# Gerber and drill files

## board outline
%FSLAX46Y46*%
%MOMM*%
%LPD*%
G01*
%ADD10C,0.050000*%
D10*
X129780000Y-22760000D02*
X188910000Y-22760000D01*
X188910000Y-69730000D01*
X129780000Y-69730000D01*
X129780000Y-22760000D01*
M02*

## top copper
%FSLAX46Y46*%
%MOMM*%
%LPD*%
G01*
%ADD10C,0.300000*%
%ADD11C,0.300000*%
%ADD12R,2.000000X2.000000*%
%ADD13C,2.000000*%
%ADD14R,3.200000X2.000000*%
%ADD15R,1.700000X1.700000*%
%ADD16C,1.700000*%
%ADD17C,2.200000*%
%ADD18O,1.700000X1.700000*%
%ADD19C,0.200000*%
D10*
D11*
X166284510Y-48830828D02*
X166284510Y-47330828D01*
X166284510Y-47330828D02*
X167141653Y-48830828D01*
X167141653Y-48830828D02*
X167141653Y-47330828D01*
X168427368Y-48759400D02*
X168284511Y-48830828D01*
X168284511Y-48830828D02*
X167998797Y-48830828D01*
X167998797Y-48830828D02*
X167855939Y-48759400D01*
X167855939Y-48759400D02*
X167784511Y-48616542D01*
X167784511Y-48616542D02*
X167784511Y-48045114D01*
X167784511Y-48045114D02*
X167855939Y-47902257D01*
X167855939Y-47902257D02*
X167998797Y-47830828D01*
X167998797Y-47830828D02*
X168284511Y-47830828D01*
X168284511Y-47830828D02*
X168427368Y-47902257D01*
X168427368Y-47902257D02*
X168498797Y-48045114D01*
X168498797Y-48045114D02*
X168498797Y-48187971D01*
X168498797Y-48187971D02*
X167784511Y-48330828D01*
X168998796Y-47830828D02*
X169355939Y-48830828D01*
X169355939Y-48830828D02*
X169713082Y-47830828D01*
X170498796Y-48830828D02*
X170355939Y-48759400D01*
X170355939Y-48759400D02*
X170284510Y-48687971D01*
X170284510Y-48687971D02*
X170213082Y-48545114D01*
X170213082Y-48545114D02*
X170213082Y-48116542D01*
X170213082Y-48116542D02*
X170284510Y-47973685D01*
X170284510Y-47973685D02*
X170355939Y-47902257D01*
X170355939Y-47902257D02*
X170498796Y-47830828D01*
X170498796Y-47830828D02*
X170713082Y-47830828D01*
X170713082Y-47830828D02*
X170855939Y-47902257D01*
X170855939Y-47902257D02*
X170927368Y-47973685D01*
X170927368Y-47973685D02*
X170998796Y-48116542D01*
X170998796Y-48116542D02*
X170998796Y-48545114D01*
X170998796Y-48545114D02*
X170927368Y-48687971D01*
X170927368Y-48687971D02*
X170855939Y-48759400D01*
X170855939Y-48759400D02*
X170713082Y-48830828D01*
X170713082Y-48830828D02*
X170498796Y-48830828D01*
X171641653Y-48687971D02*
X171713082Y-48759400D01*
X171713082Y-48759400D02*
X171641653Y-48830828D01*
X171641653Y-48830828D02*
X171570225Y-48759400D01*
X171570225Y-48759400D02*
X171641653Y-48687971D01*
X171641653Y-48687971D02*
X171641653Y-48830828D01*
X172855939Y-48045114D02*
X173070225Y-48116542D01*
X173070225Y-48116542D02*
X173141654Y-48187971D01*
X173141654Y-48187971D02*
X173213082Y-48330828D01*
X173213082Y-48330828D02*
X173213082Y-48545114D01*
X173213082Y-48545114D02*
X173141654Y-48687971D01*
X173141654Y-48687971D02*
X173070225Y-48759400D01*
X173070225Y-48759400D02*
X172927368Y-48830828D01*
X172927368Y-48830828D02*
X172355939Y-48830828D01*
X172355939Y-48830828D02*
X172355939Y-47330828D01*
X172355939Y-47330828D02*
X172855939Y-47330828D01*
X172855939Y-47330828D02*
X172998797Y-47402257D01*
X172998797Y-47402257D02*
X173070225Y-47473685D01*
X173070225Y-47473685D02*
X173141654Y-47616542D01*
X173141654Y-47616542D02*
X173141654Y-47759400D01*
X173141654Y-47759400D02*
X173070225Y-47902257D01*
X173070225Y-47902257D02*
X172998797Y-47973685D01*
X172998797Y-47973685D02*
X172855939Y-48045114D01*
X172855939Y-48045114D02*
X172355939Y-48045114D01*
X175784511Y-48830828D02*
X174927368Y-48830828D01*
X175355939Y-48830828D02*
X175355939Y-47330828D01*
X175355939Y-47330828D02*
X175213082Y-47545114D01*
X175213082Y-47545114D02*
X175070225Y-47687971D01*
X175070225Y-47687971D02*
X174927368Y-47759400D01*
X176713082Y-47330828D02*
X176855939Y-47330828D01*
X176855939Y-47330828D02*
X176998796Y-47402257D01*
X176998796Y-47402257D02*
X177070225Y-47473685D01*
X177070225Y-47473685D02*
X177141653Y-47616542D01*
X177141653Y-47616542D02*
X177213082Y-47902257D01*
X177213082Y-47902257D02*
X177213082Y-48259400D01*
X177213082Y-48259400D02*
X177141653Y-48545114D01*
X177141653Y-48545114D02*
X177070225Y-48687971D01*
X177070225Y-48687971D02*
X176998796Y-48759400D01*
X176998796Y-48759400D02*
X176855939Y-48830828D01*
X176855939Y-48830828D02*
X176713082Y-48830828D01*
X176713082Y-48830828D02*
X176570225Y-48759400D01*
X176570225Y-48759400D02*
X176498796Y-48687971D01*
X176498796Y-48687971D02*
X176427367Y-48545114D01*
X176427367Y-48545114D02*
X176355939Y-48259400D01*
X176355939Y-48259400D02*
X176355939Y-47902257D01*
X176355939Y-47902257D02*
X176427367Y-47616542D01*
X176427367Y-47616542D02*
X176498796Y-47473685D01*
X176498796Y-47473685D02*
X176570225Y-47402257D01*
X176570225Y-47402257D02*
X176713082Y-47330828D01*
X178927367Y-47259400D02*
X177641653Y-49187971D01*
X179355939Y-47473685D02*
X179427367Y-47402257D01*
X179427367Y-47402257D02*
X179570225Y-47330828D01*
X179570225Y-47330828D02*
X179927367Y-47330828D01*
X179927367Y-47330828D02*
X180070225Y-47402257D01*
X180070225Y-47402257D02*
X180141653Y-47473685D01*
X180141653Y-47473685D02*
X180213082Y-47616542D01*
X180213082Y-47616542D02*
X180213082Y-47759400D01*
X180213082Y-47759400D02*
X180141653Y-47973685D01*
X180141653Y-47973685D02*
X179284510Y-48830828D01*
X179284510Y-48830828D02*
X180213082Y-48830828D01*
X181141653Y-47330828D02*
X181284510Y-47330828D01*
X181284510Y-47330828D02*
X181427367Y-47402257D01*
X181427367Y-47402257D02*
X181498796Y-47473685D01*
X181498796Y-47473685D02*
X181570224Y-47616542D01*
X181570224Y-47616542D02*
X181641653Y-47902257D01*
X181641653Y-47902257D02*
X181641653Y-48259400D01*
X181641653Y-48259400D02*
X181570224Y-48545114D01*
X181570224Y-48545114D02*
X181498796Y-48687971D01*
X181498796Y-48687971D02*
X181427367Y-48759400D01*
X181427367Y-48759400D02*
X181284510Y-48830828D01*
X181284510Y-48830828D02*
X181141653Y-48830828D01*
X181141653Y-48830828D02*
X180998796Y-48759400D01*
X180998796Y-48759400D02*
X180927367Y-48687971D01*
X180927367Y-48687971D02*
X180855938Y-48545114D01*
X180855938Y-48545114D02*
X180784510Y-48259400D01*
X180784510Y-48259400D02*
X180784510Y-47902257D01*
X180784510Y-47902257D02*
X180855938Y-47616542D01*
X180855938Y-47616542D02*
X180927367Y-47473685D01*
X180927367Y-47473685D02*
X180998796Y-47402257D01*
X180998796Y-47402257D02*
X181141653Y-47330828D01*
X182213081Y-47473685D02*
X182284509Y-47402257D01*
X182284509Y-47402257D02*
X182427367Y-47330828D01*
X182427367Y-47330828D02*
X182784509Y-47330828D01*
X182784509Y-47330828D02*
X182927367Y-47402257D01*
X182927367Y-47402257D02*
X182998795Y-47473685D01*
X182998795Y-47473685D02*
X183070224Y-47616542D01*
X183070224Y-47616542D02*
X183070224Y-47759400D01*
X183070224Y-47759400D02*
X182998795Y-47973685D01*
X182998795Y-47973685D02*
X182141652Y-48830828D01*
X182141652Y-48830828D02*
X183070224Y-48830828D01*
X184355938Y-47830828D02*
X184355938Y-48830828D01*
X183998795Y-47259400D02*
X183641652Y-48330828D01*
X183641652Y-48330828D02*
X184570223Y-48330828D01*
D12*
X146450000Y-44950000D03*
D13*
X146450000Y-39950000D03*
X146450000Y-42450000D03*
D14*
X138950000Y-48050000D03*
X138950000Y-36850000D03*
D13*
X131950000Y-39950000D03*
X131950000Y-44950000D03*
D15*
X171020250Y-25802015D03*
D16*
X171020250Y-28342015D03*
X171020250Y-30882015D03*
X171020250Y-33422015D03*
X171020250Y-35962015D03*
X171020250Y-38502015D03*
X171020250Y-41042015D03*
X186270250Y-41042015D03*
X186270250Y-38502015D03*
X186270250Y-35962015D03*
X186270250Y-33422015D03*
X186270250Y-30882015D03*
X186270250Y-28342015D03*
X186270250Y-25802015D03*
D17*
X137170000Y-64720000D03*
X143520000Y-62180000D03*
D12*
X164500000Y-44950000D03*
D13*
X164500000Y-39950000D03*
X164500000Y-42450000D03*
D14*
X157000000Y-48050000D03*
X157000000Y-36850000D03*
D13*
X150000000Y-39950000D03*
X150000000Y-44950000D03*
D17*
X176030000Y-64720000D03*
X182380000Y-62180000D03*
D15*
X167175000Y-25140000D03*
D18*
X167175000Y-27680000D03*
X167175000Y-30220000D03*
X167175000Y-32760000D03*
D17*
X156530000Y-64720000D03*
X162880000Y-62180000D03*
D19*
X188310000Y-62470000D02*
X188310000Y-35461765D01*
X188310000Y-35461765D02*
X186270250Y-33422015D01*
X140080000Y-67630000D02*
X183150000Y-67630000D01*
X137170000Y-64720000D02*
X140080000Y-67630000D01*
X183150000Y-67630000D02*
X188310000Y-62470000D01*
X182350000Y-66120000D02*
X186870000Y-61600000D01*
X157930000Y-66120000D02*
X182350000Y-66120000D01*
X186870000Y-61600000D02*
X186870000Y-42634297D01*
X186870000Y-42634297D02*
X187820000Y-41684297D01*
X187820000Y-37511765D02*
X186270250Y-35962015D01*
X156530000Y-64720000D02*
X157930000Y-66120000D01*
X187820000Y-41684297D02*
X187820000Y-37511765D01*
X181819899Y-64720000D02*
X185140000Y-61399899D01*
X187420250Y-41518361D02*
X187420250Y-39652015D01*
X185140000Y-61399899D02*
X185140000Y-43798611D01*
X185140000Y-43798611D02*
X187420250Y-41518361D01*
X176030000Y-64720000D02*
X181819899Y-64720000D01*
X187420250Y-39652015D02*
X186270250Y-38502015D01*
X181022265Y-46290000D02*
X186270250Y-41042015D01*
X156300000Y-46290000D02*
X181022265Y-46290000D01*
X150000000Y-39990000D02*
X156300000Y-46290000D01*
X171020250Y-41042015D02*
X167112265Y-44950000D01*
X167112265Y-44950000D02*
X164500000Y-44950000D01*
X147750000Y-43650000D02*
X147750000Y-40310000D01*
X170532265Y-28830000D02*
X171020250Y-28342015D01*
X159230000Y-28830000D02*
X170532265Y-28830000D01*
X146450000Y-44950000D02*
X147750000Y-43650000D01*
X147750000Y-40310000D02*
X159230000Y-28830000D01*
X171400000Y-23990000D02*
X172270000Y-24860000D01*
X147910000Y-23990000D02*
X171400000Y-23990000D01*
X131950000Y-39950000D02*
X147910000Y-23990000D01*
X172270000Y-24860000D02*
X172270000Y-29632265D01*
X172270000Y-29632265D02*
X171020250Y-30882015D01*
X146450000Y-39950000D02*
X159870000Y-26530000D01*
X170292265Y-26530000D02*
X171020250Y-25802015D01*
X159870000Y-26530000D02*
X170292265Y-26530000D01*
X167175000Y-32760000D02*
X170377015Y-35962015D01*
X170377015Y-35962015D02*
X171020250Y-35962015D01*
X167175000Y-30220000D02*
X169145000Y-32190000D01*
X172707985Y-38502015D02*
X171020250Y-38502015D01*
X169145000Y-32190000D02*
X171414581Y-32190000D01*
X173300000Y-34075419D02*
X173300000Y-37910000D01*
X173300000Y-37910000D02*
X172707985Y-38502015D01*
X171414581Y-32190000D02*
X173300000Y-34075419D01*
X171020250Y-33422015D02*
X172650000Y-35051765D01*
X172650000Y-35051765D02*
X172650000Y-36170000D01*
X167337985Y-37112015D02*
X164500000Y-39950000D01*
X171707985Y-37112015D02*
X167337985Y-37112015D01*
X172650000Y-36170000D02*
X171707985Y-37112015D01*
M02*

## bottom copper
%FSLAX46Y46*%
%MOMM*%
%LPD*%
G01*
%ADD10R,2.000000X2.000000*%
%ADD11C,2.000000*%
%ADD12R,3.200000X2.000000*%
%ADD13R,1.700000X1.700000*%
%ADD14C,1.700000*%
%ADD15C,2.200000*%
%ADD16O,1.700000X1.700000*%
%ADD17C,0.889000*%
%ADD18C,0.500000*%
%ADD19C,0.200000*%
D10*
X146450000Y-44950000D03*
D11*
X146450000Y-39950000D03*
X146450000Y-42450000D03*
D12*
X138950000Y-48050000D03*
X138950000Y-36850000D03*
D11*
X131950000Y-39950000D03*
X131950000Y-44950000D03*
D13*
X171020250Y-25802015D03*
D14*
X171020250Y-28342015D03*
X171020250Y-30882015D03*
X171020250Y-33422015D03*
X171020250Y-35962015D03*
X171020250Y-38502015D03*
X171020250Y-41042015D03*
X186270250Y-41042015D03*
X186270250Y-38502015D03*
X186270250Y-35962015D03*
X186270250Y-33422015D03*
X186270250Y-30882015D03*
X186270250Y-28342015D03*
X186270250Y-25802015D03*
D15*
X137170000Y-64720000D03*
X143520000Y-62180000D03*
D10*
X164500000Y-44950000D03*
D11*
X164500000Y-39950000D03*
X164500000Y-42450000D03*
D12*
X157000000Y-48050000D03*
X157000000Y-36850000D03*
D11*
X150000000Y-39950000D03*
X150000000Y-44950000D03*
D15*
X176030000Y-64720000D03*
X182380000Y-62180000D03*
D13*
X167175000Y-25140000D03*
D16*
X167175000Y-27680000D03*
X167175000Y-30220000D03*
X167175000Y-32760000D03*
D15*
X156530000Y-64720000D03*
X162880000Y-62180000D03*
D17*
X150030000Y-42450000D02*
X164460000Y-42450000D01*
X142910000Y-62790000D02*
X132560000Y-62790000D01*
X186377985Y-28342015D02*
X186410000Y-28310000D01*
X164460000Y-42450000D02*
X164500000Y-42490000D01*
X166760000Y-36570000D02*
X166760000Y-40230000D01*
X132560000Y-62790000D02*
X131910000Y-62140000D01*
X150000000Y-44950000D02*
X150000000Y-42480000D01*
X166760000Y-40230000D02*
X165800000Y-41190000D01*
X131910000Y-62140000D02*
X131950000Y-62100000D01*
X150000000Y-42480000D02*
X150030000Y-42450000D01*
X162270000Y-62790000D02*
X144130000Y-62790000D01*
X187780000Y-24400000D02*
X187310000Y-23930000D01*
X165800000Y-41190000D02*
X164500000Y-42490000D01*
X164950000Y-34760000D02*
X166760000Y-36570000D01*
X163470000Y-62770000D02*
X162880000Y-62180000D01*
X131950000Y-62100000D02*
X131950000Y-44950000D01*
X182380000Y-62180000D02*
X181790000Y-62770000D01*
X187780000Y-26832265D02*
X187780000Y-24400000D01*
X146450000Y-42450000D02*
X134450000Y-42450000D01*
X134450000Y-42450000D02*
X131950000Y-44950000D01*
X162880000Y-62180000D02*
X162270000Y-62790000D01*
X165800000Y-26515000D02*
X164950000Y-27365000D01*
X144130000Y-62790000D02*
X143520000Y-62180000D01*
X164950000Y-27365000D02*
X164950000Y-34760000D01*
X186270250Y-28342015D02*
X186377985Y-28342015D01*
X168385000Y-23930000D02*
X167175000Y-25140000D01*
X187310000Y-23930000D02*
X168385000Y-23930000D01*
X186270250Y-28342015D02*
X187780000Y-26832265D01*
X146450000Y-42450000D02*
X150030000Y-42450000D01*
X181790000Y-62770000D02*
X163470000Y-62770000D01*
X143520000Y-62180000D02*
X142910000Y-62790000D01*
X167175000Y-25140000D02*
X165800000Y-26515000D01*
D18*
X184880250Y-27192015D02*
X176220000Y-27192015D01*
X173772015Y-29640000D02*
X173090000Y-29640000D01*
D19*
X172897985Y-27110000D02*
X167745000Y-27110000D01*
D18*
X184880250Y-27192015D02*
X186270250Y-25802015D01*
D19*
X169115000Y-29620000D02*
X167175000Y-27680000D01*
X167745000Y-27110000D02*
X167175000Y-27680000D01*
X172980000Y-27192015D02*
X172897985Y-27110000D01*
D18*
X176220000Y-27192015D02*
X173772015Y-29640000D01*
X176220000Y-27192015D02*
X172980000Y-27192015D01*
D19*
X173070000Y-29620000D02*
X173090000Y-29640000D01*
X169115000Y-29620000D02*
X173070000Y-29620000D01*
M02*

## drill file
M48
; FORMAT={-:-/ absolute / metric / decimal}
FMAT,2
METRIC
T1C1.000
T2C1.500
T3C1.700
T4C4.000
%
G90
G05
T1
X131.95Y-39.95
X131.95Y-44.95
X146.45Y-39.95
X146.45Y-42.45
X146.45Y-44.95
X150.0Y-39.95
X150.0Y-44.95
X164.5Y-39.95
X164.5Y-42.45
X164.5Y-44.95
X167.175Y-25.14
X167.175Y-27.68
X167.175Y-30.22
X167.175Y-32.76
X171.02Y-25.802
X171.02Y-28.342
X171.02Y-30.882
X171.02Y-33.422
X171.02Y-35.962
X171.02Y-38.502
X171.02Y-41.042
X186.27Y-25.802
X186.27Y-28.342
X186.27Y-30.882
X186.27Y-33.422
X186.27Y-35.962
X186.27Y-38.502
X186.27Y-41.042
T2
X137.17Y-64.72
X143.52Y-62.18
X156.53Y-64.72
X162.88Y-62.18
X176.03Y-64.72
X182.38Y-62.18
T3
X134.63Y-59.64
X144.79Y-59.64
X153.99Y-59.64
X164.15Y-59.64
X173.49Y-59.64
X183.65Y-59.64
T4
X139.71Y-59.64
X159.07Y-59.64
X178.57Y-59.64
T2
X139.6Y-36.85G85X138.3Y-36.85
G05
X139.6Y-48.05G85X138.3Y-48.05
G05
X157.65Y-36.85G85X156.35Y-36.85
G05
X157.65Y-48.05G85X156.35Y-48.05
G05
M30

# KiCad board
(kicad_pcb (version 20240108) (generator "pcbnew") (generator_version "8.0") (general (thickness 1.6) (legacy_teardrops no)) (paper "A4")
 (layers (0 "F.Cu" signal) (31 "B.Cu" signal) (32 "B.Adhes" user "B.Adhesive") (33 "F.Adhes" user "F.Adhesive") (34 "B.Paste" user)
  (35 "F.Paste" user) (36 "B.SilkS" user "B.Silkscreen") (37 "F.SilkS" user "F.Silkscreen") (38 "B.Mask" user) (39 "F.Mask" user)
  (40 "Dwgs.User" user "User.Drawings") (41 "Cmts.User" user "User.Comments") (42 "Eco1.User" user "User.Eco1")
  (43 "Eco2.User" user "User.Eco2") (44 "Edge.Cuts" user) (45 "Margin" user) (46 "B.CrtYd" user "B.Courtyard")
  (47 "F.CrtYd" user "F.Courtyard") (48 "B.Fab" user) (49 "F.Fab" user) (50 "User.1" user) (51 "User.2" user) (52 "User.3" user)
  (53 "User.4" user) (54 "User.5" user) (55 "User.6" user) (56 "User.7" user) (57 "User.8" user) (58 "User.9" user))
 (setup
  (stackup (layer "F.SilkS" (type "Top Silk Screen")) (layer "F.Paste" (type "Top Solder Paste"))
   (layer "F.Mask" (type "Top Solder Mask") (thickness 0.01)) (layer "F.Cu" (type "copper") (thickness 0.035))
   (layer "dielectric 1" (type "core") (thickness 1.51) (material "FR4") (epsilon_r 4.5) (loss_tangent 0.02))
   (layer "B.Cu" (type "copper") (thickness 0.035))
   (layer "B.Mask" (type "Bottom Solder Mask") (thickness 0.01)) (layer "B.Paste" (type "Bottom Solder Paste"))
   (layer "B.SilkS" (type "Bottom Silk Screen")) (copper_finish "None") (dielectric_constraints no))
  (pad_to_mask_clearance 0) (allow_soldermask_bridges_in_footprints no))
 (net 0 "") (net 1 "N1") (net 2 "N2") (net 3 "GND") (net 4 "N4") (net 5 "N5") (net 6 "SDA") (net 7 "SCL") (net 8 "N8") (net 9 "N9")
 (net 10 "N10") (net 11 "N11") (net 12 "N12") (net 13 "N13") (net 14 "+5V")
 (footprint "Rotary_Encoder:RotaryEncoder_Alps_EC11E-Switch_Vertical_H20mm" (layer "F.Cu") (at 146.45 44.95 180)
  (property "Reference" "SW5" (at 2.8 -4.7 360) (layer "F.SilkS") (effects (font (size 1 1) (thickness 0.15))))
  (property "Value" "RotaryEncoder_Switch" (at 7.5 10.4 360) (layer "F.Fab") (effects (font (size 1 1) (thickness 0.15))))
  (pad "A" thru_hole rect (at 0 0 180) (size 2 2) (drill 1) (layers "*.Cu" "*.Mask") (remove_unused_layers no) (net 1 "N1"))
  (pad "B" thru_hole circle (at 0 5 180) (size 2 2) (drill 1) (layers "*.Cu" "*.Mask") (remove_unused_layers no) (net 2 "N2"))
  (pad "C" thru_hole circle (at 0 2.5 180) (size 2 2) (drill 1) (layers "*.Cu" "*.Mask") (remove_unused_layers no) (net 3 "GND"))
  (pad "MP" thru_hole rect (at 7.5 -3.1 180) (size 3.2 2) (drill oval 2.8 1.5) (layers "*.Cu" "*.Mask") (remove_unused_layers no))
  (pad "MP" thru_hole rect (at 7.5 8.1 180) (size 3.2 2) (drill oval 2.8 1.5) (layers "*.Cu" "*.Mask") (remove_unused_layers no))
  (pad "S1" thru_hole circle (at 14.5 5 180) (size 2 2) (drill 1) (layers "*.Cu" "*.Mask") (remove_unused_layers no) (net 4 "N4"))
  (pad "S2" thru_hole circle (at 14.5 0 180) (size 2 2) (drill 1) (layers "*.Cu" "*.Mask") (remove_unused_layers no) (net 3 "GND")))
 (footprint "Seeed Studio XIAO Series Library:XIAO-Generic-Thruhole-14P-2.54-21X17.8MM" (layer "F.Cu") (at 178.64525 33.422015)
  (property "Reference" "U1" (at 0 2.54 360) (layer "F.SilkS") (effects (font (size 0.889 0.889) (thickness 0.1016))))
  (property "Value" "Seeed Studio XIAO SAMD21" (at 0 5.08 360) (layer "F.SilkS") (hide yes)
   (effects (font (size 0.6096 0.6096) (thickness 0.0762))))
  (pad "1" thru_hole rect (at -7.625 -7.62) (size 1.7 1.7) (drill 1) (layers "*.Cu" "*.Mask") (remove_unused_layers no) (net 2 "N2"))
  (pad "2" thru_hole circle (at -7.625 -5.08) (size 1.7 1.7) (drill 1) (layers "*.Cu" "*.Mask") (remove_unused_layers no) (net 1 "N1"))
  (pad "3" thru_hole circle (at -7.625 -2.54) (size 1.7 1.7) (drill 1) (layers "*.Cu" "*.Mask") (remove_unused_layers no) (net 4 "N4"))
  (pad "4" thru_hole circle (at -7.625 0) (size 1.7 1.7) (drill 1) (layers "*.Cu" "*.Mask") (remove_unused_layers no) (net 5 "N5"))
  (pad "5" thru_hole circle (at -7.625 2.54) (size 1.7 1.7) (drill 1) (layers "*.Cu" "*.Mask") (remove_unused_layers no) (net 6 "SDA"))
  (pad "6" thru_hole circle (at -7.625 5.08 180) (size 1.7 1.7) (drill 1) (layers "*.Cu" "*.Mask") (remove_unused_layers no) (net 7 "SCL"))
  (pad "7" thru_hole circle (at -7.625 7.62) (size 1.7 1.7) (drill 1) (layers "*.Cu" "*.Mask") (remove_unused_layers no) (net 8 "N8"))
  (pad "8" thru_hole circle (at 7.625 7.62) (size 1.7 1.7) (drill 1) (layers "*.Cu" "*.Mask") (remove_unused_layers no) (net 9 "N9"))
  (pad "9" thru_hole circle (at 7.625 5.08) (size 1.7 1.7) (drill 1) (layers "*.Cu" "*.Mask") (remove_unused_layers no) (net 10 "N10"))
  (pad "10" thru_hole circle (at 7.625 2.54) (size 1.7 1.7) (drill 1) (layers "*.Cu" "*.Mask") (remove_unused_layers no) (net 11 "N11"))
  (pad "11" thru_hole circle (at 7.625 0) (size 1.7 1.7) (drill 1) (layers "*.Cu" "*.Mask") (remove_unused_layers no) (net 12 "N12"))
  (pad "12" thru_hole circle (at 7.625 -2.54) (size 1.7 1.7) (drill 1) (layers "*.Cu" "*.Mask") (remove_unused_layers no) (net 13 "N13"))
  (pad "13" thru_hole circle (at 7.625 -5.08) (size 1.7 1.7) (drill 1) (layers "*.Cu" "*.Mask") (remove_unused_layers no) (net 3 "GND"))
  (pad "14" thru_hole circle (at 7.625 -7.62) (size 1.7 1.7) (drill 1) (layers "*.Cu" "*.Mask") (remove_unused_layers no) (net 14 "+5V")))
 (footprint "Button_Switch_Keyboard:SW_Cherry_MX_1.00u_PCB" (layer "F.Cu") (at 137.17 64.72 180)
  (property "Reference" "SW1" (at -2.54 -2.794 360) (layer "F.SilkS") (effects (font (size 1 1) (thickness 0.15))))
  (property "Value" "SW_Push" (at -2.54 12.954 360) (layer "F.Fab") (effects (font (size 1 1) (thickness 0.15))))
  (pad "" np_thru_hole circle (at -7.62 5.08 180) (size 1.7 1.7) (drill 1.7) (layers "*.Cu" "*.Mask"))
  (pad "" np_thru_hole circle (at -2.54 5.08 180) (size 4 4) (drill 4) (layers "*.Cu" "*.Mask"))
  (pad "" np_thru_hole circle (at 2.54 5.08 180) (size 1.7 1.7) (drill 1.7) (layers "*.Cu" "*.Mask"))
  (pad "1" thru_hole circle (at 0 0 180) (size 2.2 2.2) (drill 1.5) (layers "*.Cu" "*.Mask") (remove_unused_layers no) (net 12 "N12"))
  (pad "2" thru_hole circle (at -6.35 2.54 180) (size 2.2 2.2) (drill 1.5) (layers "*.Cu" "*.Mask") (remove_unused_layers no) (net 3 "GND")))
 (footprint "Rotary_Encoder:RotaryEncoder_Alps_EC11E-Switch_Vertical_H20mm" (layer "F.Cu") (at 164.5 44.95 180)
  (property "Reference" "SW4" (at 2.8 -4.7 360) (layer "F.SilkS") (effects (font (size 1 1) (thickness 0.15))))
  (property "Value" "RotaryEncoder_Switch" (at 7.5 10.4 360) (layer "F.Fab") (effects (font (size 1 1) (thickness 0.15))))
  (pad "A" thru_hole rect (at 0 0 180) (size 2 2) (drill 1) (layers "*.Cu" "*.Mask") (remove_unused_layers no) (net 8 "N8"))
  (pad "B" thru_hole circle (at 0 5 180) (size 2 2) (drill 1) (layers "*.Cu" "*.Mask") (remove_unused_layers no) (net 5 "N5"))
  (pad "C" thru_hole circle (at 0 2.5 180) (size 2 2) (drill 1) (layers "*.Cu" "*.Mask") (remove_unused_layers no) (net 3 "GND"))
  (pad "MP" thru_hole rect (at 7.5 -3.1 180) (size 3.2 2) (drill oval 2.8 1.5) (layers "*.Cu" "*.Mask") (remove_unused_layers no))
  (pad "MP" thru_hole rect (at 7.5 8.1 180) (size 3.2 2) (drill oval 2.8 1.5) (layers "*.Cu" "*.Mask") (remove_unused_layers no))
  (pad "S1" thru_hole circle (at 14.5 5 180) (size 2 2) (drill 1) (layers "*.Cu" "*.Mask") (remove_unused_layers no) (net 9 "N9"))
  (pad "S2" thru_hole circle (at 14.5 0 180) (size 2 2) (drill 1) (layers "*.Cu" "*.Mask") (remove_unused_layers no) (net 3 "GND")))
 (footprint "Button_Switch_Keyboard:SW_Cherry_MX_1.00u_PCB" (layer "F.Cu") (at 176.03 64.72 180)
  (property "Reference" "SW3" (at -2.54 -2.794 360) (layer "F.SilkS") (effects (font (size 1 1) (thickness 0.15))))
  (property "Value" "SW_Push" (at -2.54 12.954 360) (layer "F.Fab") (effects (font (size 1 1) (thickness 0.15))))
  (pad "" np_thru_hole circle (at -7.62 5.08 180) (size 1.7 1.7) (drill 1.7) (layers "*.Cu" "*.Mask"))
  (pad "" np_thru_hole circle (at -2.54 5.08 180) (size 4 4) (drill 4) (layers "*.Cu" "*.Mask"))
  (pad "" np_thru_hole circle (at 2.54 5.08 180) (size 1.7 1.7) (drill 1.7) (layers "*.Cu" "*.Mask"))
  (pad "1" thru_hole circle (at 0 0 180) (size 2.2 2.2) (drill 1.5) (layers "*.Cu" "*.Mask") (remove_unused_layers no) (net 10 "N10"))
  (pad "2" thru_hole circle (at -6.35 2.54 180) (size 2.2 2.2) (drill 1.5) (layers "*.Cu" "*.Mask") (remove_unused_layers no) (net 3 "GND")))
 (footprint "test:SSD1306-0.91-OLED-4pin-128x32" (layer "F.Cu") (at 130.675 22.95)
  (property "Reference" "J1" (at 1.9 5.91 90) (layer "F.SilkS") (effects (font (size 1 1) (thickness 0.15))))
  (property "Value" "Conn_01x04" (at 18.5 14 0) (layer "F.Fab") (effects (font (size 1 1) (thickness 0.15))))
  (pad "1" thru_hole rect (at 36.5 2.19) (size 1.7 1.7) (drill 1) (layers "*.Cu" "*.Mask") (remove_unused_layers no) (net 3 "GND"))
  (pad "2" thru_hole oval (at 36.5 4.73) (size 1.7 1.7) (drill 1) (layers "*.Cu" "*.Mask") (remove_unused_layers no) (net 14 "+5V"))
  (pad "3" thru_hole oval (at 36.5 7.27) (size 1.7 1.7) (drill 1) (layers "*.Cu" "*.Mask") (remove_unused_layers no) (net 7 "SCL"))
  (pad "4" thru_hole oval (at 36.5 9.81) (size 1.7 1.7) (drill 1) (layers "*.Cu" "*.Mask") (remove_unused_layers no) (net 6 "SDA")))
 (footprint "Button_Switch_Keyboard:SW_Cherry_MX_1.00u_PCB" (layer "F.Cu") (at 156.53 64.72 180)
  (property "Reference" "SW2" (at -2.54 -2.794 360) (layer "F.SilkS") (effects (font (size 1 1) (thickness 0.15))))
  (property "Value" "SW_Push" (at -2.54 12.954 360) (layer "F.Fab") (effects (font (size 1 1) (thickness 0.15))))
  (pad "" np_thru_hole circle (at -7.62 5.08 180) (size 1.7 1.7) (drill 1.7) (layers "*.Cu" "*.Mask"))
  (pad "" np_thru_hole circle (at -2.54 5.08 180) (size 4 4) (drill 4) (layers "*.Cu" "*.Mask"))
  (pad "" np_thru_hole circle (at 2.54 5.08 180) (size 1.7 1.7) (drill 1.7) (layers "*.Cu" "*.Mask"))
  (pad "1" thru_hole circle (at 0 0 180) (size 2.2 2.2) (drill 1.5) (layers "*.Cu" "*.Mask") (remove_unused_layers no) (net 11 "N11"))
  (pad "2" thru_hole circle (at -6.35 2.54 180) (size 2.2 2.2) (drill 1.5) (layers "*.Cu" "*.Mask") (remove_unused_layers no) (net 3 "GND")))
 (gr_rect (start 129.78 22.76) (end 188.91 69.73) (stroke (width 0.05) (type default)) (fill none) (layer "Edge.Cuts"))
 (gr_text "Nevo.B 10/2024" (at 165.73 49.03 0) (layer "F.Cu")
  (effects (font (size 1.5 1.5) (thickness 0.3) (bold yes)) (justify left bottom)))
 (segment (start 150.03 42.45) (end 164.46 42.45) (width 0.889) (layer "B.Cu") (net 3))
 (segment (start 142.91 62.79) (end 132.56 62.79) (width 0.889) (layer "B.Cu") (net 3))
 (segment (start 186.377985 28.342015) (end 186.41 28.31) (width 0.889) (layer "B.Cu") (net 3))
 (segment (start 164.46 42.45) (end 164.5 42.49) (width 0.889) (layer "B.Cu") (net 3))
 (segment (start 166.76 36.57) (end 166.76 40.23) (width 0.889) (layer "B.Cu") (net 3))
 (segment (start 132.56 62.79) (end 131.91 62.14) (width 0.889) (layer "B.Cu") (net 3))
 (segment (start 150 44.95) (end 150 42.48) (width 0.889) (layer "B.Cu") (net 3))
 (segment (start 166.76 40.23) (end 165.8 41.19) (width 0.889) (layer "B.Cu") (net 3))
 (segment (start 131.91 62.14) (end 131.95 62.1) (width 0.889) (layer "B.Cu") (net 3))
 (segment (start 150 42.48) (end 150.03 42.45) (width 0.889) (layer "B.Cu") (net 3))
 (segment (start 162.27 62.79) (end 144.13 62.79) (width 0.889) (layer "B.Cu") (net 3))
 (segment (start 187.78 24.4) (end 187.31 23.93) (width 0.889) (layer "B.Cu") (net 3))
 (segment (start 165.8 41.19) (end 164.5 42.49) (width 0.889) (layer "B.Cu") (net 3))
 (segment (start 164.95 34.76) (end 166.76 36.57) (width 0.889) (layer "B.Cu") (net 3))
 (segment (start 163.47 62.77) (end 162.88 62.18) (width 0.889) (layer "B.Cu") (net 3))
 (segment (start 131.95 62.1) (end 131.95 44.95) (width 0.889) (layer "B.Cu") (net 3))
 (segment (start 182.38 62.18) (end 181.79 62.77) (width 0.889) (layer "B.Cu") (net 3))
 (segment (start 187.78 26.832265) (end 187.78 24.4) (width 0.889) (layer "B.Cu") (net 3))
 (segment (start 146.45 42.45) (end 134.45 42.45) (width 0.889) (layer "B.Cu") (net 3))
 (segment (start 134.45 42.45) (end 131.95 44.95) (width 0.889) (layer "B.Cu") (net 3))
 (segment (start 162.88 62.18) (end 162.27 62.79) (width 0.889) (layer "B.Cu") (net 3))
 (segment (start 165.8 26.515) (end 164.95 27.365) (width 0.889) (layer "B.Cu") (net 3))
 (segment (start 144.13 62.79) (end 143.52 62.18) (width 0.889) (layer "B.Cu") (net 3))
 (segment (start 164.95 27.365) (end 164.95 34.76) (width 0.889) (layer "B.Cu") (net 3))
 (segment (start 186.27025 28.342015) (end 186.377985 28.342015) (width 0.889) (layer "B.Cu") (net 3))
 (segment (start 168.385 23.93) (end 167.175 25.14) (width 0.889) (layer "B.Cu") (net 3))
 (segment (start 187.31 23.93) (end 168.385 23.93) (width 0.889) (layer "B.Cu") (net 3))
 (segment (start 186.27025 28.342015) (end 187.78 26.832265) (width 0.889) (layer "B.Cu") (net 3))
 (segment (start 146.45 42.45) (end 150.03 42.45) (width 0.889) (layer "B.Cu") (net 3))
 (segment (start 181.79 62.77) (end 163.47 62.77) (width 0.889) (layer "B.Cu") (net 3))
 (segment (start 143.52 62.18) (end 142.91 62.79) (width 0.889) (layer "B.Cu") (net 3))
 (segment (start 167.175 25.14) (end 165.8 26.515) (width 0.889) (layer "B.Cu") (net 3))
 (segment (start 188.31 62.47) (end 188.31 35.461765) (width 0.2) (layer "F.Cu") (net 12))
 (segment (start 188.31 35.461765) (end 186.27025 33.422015) (width 0.2) (layer "F.Cu") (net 12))
 (segment (start 140.08 67.63) (end 183.15 67.63) (width 0.2) (layer "F.Cu") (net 12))
 (segment (start 137.17 64.72) (end 140.08 67.63) (width 0.2) (layer "F.Cu") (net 12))
 (segment (start 183.15 67.63) (end 188.31 62.47) (width 0.2) (layer "F.Cu") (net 12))
 (segment (start 182.35 66.12) (end 186.87 61.6) (width 0.2) (layer "F.Cu") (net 11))
 (segment (start 157.93 66.12) (end 182.35 66.12) (width 0.2) (layer "F.Cu") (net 11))
 (segment (start 186.87 61.6) (end 186.87 42.634297) (width 0.2) (layer "F.Cu") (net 11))
 (segment (start 186.87 42.634297) (end 187.82 41.684297) (width 0.2) (layer "F.Cu") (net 11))
 (segment (start 187.82 37.511765) (end 186.27025 35.962015) (width 0.2) (layer "F.Cu") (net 11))
 (segment (start 156.53 64.72) (end 157.93 66.12) (width 0.2) (layer "F.Cu") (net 11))
 (segment (start 187.82 41.684297) (end 187.82 37.511765) (width 0.2) (layer "F.Cu") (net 11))
 (segment (start 181.819899 64.72) (end 185.14 61.399899) (width 0.2) (layer "F.Cu") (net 10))
 (segment (start 187.42025 41.518361) (end 187.42025 39.652015) (width 0.2) (layer "F.Cu") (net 10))
 (segment (start 185.14 61.399899) (end 185.14 43.798611) (width 0.2) (layer "F.Cu") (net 10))
 (segment (start 185.14 43.798611) (end 187.42025 41.518361) (width 0.2) (layer "F.Cu") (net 10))
 (segment (start 176.03 64.72) (end 181.819899 64.72) (width 0.2) (layer "F.Cu") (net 10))
 (segment (start 187.42025 39.652015) (end 186.27025 38.502015) (width 0.2) (layer "F.Cu") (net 10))
 (segment (start 181.022265 46.29) (end 186.27025 41.042015) (width 0.2) (layer "F.Cu") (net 9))
 (segment (start 156.3 46.29) (end 181.022265 46.29) (width 0.2) (layer "F.Cu") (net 9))
 (segment (start 150 39.99) (end 156.3 46.29) (width 0.2) (layer "F.Cu") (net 9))
 (segment (start 171.02025 41.042015) (end 167.112265 44.95) (width 0.2) (layer "F.Cu") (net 8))
 (segment (start 167.112265 44.95) (end 164.5 44.95) (width 0.2) (layer "F.Cu") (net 8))
 (segment (start 147.75 43.65) (end 147.75 40.31) (width 0.2) (layer "F.Cu") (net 1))
 (segment (start 170.532265 28.83) (end 171.02025 28.342015) (width 0.2) (layer "F.Cu") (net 1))
 (segment (start 159.23 28.83) (end 170.532265 28.83) (width 0.2) (layer "F.Cu") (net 1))
 (segment (start 146.45 44.95) (end 147.75 43.65) (width 0.2) (layer "F.Cu") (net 1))
 (segment (start 147.75 40.31) (end 159.23 28.83) (width 0.2) (layer "F.Cu") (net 1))
 (segment (start 171.4 23.99) (end 172.27 24.86) (width 0.2) (layer "F.Cu") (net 4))
 (segment (start 147.91 23.99) (end 171.4 23.99) (width 0.2) (layer "F.Cu") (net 4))
 (segment (start 131.95 39.95) (end 147.91 23.99) (width 0.2) (layer "F.Cu") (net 4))
 (segment (start 172.27 24.86) (end 172.27 29.632265) (width 0.2) (layer "F.Cu") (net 4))
 (segment (start 172.27 29.632265) (end 171.02025 30.882015) (width 0.2) (layer "F.Cu") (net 4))
 (segment (start 146.45 39.95) (end 159.87 26.53) (width 0.2) (layer "F.Cu") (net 2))
 (segment (start 170.292265 26.53) (end 171.02025 25.802015) (width 0.2) (layer "F.Cu") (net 2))
 (segment (start 159.87 26.53) (end 170.292265 26.53) (width 0.2) (layer "F.Cu") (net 2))
 (segment (start 184.88025 27.192015) (end 176.22 27.192015) (width 0.5) (layer "B.Cu") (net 14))
 (segment (start 173.772015 29.64) (end 173.09 29.64) (width 0.5) (layer "B.Cu") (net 14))
 (segment (start 172.897985 27.11) (end 167.745 27.11) (width 0.2) (layer "B.Cu") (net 14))
 (segment (start 184.88025 27.192015) (end 186.27025 25.802015) (width 0.5) (layer "B.Cu") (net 14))
 (segment (start 169.115 29.62) (end 167.175 27.68) (width 0.2) (layer "B.Cu") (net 14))
 (segment (start 167.745 27.11) (end 167.175 27.68) (width 0.2) (layer "B.Cu") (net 14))
 (segment (start 172.98 27.192015) (end 172.897985 27.11) (width 0.2) (layer "B.Cu") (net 14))
 (segment (start 176.22 27.192015) (end 173.772015 29.64) (width 0.5) (layer "B.Cu") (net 14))
 (segment (start 176.22 27.192015) (end 172.98 27.192015) (width 0.5) (layer "B.Cu") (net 14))
 (segment (start 173.07 29.62) (end 173.09 29.64) (width 0.2) (layer "B.Cu") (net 14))
 (segment (start 169.115 29.62) (end 173.07 29.62) (width 0.2) (layer "B.Cu") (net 14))
 (segment (start 167.175 32.76) (end 170.377015 35.962015) (width 0.2) (layer "F.Cu") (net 6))
 (segment (start 170.377015 35.962015) (end 171.02025 35.962015) (width 0.2) (layer "F.Cu") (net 6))
 (segment (start 167.175 30.22) (end 169.145 32.19) (width 0.2) (layer "F.Cu") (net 7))
 (segment (start 172.707985 38.502015) (end 171.02025 38.502015) (width 0.2) (layer "F.Cu") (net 7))
 (segment (start 169.145 32.19) (end 171.414581 32.19) (width 0.2) (layer "F.Cu") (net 7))
 (segment (start 173.3 34.075419) (end 173.3 37.91) (width 0.2) (layer "F.Cu") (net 7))
 (segment (start 173.3 37.91) (end 172.707985 38.502015) (width 0.2) (layer "F.Cu") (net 7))
 (segment (start 171.414581 32.19) (end 173.3 34.075419) (width 0.2) (layer "F.Cu") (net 7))
 (segment (start 171.02025 33.422015) (end 172.65 35.051765) (width 0.2) (layer "F.Cu") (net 5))
 (segment (start 172.65 35.051765) (end 172.65 36.17) (width 0.2) (layer "F.Cu") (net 5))
 (segment (start 167.337985 37.112015) (end 164.5 39.95) (width 0.2) (layer "F.Cu") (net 5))
 (segment (start 171.707985 37.112015) (end 167.337985 37.112015) (width 0.2) (layer "F.Cu") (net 5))
 (segment (start 172.65 36.17) (end 171.707985 37.112015) (width 0.2) (layer "F.Cu") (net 5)))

